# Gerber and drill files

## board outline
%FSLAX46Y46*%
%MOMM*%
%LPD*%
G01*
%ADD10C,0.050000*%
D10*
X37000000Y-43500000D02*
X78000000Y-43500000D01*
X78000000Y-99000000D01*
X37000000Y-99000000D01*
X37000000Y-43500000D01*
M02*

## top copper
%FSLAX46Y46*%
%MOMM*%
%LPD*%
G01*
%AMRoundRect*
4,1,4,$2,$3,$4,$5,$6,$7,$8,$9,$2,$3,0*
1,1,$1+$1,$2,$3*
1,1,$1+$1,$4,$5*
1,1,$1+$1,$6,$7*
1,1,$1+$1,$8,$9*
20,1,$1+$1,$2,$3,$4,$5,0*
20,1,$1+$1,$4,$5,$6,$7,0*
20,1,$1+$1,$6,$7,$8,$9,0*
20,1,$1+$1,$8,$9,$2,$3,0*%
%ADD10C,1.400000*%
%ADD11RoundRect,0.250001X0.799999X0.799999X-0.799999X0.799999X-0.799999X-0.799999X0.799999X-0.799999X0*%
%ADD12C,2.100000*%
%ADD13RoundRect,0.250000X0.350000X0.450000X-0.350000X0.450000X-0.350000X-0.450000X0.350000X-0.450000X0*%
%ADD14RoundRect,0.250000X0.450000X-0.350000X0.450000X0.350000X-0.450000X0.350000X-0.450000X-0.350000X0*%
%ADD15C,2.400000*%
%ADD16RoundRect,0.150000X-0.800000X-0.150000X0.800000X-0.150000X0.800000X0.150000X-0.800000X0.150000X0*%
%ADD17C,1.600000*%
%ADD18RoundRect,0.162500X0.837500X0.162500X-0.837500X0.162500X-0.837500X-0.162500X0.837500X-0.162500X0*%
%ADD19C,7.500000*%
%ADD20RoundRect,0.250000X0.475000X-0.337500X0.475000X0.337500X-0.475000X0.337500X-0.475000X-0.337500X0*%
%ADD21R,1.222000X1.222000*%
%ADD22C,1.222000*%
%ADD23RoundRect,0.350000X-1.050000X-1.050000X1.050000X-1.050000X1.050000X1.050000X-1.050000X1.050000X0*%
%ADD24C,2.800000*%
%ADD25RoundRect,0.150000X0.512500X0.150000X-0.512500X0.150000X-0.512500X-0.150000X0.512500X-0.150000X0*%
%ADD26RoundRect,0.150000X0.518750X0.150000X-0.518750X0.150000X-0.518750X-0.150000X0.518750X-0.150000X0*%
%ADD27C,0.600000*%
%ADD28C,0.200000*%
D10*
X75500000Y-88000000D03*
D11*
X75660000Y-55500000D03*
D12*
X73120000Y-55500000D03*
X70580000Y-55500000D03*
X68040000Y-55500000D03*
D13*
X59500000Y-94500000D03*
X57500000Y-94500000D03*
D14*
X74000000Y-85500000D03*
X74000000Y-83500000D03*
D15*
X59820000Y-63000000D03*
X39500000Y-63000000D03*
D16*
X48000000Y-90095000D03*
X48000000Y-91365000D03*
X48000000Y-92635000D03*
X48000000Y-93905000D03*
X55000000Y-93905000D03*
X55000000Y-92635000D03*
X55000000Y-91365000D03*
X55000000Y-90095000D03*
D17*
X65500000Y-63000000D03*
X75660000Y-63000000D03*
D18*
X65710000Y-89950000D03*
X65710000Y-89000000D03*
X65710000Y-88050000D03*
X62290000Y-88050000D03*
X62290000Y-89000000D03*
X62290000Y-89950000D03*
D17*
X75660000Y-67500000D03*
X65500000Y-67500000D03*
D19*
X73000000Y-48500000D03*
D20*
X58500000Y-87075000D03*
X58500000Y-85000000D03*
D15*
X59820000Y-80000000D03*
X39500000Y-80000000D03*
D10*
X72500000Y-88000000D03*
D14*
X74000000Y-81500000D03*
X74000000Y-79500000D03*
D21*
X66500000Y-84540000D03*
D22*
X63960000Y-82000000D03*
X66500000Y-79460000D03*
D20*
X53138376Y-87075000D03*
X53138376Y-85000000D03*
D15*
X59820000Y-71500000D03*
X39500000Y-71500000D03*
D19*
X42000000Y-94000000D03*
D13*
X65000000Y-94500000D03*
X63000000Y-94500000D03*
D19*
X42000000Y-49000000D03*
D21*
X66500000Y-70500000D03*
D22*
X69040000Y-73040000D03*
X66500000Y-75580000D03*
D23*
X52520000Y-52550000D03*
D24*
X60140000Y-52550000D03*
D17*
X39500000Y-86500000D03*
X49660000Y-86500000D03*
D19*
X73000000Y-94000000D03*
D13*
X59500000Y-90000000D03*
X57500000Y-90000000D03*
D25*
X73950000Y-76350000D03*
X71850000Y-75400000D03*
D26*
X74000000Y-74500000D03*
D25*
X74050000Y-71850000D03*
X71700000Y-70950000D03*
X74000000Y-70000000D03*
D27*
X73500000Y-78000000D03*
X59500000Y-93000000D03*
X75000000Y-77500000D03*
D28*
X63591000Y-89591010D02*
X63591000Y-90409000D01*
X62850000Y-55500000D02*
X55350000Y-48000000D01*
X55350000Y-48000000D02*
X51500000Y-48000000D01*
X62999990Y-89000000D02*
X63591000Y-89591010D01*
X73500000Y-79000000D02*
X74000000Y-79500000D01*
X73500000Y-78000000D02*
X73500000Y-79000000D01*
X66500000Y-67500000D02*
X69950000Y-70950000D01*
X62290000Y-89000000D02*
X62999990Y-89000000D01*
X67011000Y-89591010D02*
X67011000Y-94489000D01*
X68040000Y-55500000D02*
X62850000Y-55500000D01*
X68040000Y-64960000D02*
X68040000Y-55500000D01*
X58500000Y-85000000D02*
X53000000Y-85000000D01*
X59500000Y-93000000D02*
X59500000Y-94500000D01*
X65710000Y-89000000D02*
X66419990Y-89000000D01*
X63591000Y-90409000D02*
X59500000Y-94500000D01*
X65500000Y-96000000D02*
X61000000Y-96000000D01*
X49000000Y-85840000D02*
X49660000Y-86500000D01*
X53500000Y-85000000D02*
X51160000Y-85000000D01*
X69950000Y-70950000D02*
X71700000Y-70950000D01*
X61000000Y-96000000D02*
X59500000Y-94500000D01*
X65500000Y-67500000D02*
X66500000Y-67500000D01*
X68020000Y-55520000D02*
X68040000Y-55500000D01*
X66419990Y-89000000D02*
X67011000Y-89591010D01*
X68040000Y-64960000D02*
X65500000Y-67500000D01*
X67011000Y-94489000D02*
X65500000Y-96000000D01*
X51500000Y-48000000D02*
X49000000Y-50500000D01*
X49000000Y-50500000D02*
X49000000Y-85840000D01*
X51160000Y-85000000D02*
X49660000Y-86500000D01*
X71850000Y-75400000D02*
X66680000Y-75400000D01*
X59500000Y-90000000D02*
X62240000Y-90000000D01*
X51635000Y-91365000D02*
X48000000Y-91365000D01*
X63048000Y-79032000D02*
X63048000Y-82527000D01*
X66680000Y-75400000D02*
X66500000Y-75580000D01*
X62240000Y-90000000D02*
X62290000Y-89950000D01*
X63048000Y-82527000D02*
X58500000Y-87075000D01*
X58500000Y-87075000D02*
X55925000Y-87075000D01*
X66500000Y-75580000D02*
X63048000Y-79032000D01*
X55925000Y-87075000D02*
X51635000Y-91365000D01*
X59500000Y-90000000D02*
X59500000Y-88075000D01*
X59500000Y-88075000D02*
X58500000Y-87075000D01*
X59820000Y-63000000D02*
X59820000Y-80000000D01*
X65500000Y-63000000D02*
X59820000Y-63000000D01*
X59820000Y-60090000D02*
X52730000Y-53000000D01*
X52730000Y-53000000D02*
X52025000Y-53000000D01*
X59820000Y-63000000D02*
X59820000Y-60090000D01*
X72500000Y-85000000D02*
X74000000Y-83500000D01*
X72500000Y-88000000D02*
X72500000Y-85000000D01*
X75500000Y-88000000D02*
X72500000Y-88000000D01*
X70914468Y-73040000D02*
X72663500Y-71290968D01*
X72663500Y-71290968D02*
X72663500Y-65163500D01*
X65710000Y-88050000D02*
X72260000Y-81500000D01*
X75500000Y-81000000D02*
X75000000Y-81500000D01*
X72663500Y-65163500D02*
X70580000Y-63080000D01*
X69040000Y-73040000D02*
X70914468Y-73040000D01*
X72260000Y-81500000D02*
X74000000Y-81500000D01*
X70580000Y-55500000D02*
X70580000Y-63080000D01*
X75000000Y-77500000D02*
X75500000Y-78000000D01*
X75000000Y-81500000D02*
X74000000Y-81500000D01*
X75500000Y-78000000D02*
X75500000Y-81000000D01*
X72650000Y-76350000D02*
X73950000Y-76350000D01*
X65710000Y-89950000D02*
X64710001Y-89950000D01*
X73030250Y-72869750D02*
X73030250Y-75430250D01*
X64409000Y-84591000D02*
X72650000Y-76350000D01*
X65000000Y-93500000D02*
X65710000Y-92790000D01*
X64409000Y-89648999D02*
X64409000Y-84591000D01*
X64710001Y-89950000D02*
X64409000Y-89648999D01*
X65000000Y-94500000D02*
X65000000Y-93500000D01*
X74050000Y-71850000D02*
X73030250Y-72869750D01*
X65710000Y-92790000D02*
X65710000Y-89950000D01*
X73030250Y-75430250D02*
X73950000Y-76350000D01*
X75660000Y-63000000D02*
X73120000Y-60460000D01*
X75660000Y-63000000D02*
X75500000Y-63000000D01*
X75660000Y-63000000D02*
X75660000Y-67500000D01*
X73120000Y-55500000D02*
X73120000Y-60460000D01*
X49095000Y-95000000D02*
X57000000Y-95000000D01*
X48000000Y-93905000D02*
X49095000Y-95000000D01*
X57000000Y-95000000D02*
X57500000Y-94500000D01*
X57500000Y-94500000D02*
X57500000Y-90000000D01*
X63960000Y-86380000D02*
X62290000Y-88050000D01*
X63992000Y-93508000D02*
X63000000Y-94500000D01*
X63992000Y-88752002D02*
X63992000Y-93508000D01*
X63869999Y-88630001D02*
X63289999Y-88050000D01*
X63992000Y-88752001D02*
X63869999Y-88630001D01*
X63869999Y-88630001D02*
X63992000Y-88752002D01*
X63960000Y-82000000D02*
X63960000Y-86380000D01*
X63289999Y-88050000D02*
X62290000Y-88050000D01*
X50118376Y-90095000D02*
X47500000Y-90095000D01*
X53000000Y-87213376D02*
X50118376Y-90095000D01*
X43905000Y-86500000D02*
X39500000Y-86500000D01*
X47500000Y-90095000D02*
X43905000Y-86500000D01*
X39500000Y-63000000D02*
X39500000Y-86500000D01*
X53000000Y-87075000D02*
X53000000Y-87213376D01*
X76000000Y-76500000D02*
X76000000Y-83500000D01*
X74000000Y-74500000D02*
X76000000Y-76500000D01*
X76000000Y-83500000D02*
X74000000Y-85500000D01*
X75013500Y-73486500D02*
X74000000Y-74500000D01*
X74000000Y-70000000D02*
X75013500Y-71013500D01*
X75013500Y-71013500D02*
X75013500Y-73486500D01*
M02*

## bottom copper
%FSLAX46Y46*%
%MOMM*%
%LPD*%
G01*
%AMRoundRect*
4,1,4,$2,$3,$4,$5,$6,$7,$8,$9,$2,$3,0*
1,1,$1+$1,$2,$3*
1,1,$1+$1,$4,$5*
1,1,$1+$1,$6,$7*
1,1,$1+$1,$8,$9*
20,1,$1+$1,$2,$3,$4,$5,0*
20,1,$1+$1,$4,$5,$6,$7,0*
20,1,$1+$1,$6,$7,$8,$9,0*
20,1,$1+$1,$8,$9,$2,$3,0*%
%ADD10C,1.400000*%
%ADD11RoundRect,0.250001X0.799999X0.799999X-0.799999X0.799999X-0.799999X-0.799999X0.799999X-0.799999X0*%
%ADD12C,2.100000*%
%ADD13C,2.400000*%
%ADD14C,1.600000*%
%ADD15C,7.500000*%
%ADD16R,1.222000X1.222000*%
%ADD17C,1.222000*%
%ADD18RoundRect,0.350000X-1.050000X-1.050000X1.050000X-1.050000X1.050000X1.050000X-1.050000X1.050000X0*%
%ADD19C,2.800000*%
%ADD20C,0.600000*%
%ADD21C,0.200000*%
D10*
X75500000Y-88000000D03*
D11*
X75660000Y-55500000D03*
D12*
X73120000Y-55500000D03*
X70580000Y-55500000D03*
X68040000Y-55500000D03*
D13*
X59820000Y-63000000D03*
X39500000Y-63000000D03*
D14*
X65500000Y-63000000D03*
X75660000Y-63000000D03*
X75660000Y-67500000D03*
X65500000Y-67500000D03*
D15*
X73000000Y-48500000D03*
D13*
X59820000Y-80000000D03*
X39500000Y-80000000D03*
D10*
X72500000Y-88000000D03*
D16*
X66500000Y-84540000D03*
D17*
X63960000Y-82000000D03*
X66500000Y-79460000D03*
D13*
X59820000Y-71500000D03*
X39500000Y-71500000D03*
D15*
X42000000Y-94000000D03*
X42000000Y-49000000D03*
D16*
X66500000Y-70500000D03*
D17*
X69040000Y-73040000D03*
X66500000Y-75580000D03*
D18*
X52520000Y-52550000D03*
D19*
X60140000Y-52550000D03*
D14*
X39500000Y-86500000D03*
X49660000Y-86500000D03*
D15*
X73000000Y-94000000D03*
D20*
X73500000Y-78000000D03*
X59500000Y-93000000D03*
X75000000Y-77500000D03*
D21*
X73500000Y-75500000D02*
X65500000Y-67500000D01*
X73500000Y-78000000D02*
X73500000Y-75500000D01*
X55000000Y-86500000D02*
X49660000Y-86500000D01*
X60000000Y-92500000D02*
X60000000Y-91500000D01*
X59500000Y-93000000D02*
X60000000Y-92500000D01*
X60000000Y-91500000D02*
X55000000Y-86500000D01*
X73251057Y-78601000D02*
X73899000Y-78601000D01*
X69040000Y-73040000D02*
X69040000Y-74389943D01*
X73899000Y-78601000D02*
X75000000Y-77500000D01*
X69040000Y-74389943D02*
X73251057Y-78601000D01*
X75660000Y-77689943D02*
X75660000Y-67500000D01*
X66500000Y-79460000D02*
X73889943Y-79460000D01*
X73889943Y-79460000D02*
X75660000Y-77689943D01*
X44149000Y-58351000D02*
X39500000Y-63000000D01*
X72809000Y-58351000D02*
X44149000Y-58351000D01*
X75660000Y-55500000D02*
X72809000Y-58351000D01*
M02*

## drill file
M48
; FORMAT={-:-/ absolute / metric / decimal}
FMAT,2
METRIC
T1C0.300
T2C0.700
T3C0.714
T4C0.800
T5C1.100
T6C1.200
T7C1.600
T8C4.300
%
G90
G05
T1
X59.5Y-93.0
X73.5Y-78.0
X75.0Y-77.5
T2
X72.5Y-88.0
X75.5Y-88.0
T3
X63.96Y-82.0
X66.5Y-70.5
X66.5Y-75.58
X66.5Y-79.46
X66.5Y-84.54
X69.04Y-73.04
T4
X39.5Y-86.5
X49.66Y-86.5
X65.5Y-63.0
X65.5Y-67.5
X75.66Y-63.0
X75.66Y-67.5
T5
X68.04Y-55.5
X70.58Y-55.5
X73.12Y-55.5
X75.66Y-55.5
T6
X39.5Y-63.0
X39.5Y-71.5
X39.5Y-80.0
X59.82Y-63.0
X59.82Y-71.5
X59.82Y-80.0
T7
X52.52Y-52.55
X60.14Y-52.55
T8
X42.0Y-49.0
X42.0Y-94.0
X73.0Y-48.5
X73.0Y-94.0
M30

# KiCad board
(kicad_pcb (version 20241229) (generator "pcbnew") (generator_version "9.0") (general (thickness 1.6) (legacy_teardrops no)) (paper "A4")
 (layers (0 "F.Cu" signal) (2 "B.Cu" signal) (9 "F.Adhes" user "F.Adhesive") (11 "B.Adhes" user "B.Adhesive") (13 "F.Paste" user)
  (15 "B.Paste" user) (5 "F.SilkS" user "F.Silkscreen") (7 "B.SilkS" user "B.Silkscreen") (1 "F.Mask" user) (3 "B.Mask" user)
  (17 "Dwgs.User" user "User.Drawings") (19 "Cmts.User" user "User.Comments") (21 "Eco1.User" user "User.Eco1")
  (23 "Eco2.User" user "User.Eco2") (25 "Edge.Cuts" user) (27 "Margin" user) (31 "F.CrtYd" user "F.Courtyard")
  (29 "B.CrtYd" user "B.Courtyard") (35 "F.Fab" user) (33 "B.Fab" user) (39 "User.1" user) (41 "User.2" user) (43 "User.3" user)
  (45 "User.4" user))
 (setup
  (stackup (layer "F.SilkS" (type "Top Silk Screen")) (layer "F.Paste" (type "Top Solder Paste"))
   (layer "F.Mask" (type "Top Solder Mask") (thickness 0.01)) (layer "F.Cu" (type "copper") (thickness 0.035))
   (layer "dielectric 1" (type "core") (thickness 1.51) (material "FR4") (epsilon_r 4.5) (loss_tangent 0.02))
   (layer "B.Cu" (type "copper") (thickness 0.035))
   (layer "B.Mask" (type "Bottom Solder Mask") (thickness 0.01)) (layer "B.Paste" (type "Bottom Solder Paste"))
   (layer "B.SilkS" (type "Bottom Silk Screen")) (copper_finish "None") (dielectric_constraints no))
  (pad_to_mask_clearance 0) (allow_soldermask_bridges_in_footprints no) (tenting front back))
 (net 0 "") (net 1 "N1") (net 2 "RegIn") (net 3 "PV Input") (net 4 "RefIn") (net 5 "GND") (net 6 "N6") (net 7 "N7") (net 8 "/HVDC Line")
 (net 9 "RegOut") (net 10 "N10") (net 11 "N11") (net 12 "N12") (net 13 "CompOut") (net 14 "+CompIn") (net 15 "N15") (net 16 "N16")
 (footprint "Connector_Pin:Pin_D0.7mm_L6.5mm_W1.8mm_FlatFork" (layer "F.Cu") (at 75.5 88)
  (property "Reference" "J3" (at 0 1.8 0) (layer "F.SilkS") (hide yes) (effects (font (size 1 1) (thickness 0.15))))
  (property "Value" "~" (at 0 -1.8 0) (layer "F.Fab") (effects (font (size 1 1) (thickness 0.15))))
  (pad "1" thru_hole circle (at 0 0) (size 1.4 1.4) (drill 0.7) (layers "*.Cu" "*.Mask") (remove_unused_layers no) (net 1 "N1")))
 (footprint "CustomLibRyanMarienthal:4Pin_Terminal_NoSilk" (layer "F.Cu") (at 71.85 55.54 180)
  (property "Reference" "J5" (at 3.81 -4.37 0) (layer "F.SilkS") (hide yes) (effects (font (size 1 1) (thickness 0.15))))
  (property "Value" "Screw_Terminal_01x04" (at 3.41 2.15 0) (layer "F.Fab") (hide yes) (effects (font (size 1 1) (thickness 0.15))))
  (pad "1" thru_hole roundrect (at -3.81 0.04 180) (size 2.1 2.1) (drill 1.1) (layers "*.Cu" "*.Mask") (remove_unused_layers no)
   (roundrect_rratio 0.119048) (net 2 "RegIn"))
  (pad "2" thru_hole circle (at -1.27 0.04 180) (size 2.1 2.1) (drill 1.1) (layers "*.Cu" "*.Mask") (remove_unused_layers no)
   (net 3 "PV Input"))
  (pad "3" thru_hole circle (at 1.27 0.04 180) (size 2.1 2.1) (drill 1.1) (layers "*.Cu" "*.Mask") (remove_unused_layers no) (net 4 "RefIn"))
  (pad "4" thru_hole circle (at 3.81 0.04 180) (size 2.1 2.1) (drill 1.1) (layers "*.Cu" "*.Mask") (remove_unused_layers no) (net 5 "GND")))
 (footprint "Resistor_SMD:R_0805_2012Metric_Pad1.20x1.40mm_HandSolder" (layer "F.Cu") (at 58.5 94.5 180)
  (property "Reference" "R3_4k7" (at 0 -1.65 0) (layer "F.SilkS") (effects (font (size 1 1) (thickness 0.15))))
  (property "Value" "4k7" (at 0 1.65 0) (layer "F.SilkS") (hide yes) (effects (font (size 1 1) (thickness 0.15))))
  (pad "1" smd roundrect (at -1 0 180) (size 1.2 1.4) (layers "F.Cu" "F.Mask" "F.Paste") (roundrect_rratio 0.208333) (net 5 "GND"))
  (pad "2" smd roundrect (at 1 0 180) (size 1.2 1.4) (layers "F.Cu" "F.Mask" "F.Paste") (roundrect_rratio 0.208333) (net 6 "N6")))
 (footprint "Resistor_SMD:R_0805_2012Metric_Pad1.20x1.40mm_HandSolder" (layer "F.Cu") (at 74 84.5 90)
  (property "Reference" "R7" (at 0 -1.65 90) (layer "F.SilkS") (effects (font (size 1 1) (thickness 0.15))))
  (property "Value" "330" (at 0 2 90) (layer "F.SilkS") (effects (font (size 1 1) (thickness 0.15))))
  (pad "1" smd roundrect (at -1 0 90) (size 1.2 1.4) (layers "F.Cu" "F.Mask" "F.Paste") (roundrect_rratio 0.208333) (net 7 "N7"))
  (pad "2" smd roundrect (at 1 0 90) (size 1.2 1.4) (layers "F.Cu" "F.Mask" "F.Paste") (roundrect_rratio 0.208333) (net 1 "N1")))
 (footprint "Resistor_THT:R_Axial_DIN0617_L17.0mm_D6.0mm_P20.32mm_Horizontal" (layer "F.Cu") (at 59.82 63 180)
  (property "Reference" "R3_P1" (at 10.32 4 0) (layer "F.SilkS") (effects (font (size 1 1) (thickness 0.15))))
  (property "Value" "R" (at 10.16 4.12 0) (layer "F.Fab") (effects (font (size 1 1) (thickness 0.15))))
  (pad "1" thru_hole circle (at 0 0 180) (size 2.4 2.4) (drill 1.2) (layers "*.Cu" "*.Mask") (remove_unused_layers no) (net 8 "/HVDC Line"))
  (pad "2" thru_hole circle (at 20.32 0 180) (size 2.4 2.4) (drill 1.2) (layers "*.Cu" "*.Mask") (remove_unused_layers no) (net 2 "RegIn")))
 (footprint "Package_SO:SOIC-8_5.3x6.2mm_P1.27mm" (layer "F.Cu") (at 51.5 92)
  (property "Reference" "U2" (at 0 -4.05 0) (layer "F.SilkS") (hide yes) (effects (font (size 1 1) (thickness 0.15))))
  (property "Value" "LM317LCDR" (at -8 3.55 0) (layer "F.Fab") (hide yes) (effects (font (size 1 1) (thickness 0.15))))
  (pad "1" smd roundrect (at -3.5 -1.905) (size 1.9 0.6) (layers "F.Cu" "F.Mask" "F.Paste") (roundrect_rratio 0.25) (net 2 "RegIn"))
  (pad "2" smd roundrect (at -3.5 -0.635) (size 1.9 0.6) (layers "F.Cu" "F.Mask" "F.Paste") (roundrect_rratio 0.25) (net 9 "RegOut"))
  (pad "3" smd roundrect (at -3.5 0.635) (size 1.9 0.6) (layers "F.Cu" "F.Mask" "F.Paste") (roundrect_rratio 0.25) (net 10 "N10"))
  (pad "4" smd roundrect (at -3.5 1.905) (size 1.9 0.6) (layers "F.Cu" "F.Mask" "F.Paste") (roundrect_rratio 0.25) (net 6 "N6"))
  (pad "5" smd roundrect (at 3.5 1.905) (size 1.9 0.6) (layers "F.Cu" "F.Mask" "F.Paste") (roundrect_rratio 0.25))
  (pad "6" smd roundrect (at 3.5 0.635) (size 1.9 0.6) (layers "F.Cu" "F.Mask" "F.Paste") (roundrect_rratio 0.25) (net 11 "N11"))
  (pad "7" smd roundrect (at 3.5 -0.635) (size 1.9 0.6) (layers "F.Cu" "F.Mask" "F.Paste") (roundrect_rratio 0.25) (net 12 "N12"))
  (pad "8" smd roundrect (at 3.5 -1.905) (size 1.9 0.6) (layers "F.Cu" "F.Mask" "F.Paste") (roundrect_rratio 0.25)))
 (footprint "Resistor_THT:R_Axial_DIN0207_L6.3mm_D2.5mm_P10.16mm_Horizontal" (layer "F.Cu") (at 65.5 63)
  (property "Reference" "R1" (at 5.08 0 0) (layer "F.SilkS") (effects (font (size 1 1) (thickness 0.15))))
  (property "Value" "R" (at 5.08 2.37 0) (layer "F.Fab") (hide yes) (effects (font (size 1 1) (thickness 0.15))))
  (pad "1" thru_hole circle (at 0 0) (size 1.6 1.6) (drill 0.8) (layers "*.Cu" "*.Mask") (remove_unused_layers no) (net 8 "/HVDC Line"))
  (pad "2" thru_hole circle (at 10.16 0) (size 1.6 1.6) (drill 0.8) (layers "*.Cu" "*.Mask") (remove_unused_layers no) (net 3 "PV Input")))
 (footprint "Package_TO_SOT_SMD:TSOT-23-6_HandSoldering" (layer "F.Cu") (at 64 89 180)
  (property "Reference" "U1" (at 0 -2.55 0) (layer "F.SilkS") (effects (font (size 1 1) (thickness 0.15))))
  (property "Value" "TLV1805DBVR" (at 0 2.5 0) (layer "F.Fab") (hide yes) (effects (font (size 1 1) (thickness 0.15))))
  (pad "1" smd roundrect (at -1.71 -0.95 180) (size 2 0.65) (layers "F.Cu" "F.Mask" "F.Paste") (roundrect_rratio 0.25) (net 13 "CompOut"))
  (pad "2" smd roundrect (at -1.71 0 180) (size 2 0.65) (layers "F.Cu" "F.Mask" "F.Paste") (roundrect_rratio 0.25) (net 5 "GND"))
  (pad "3" smd roundrect (at -1.71 0.95 180) (size 2 0.65) (layers "F.Cu" "F.Mask" "F.Paste") (roundrect_rratio 0.25) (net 4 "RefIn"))
  (pad "4" smd roundrect (at 1.71 0.95 180) (size 2 0.65) (layers "F.Cu" "F.Mask" "F.Paste") (roundrect_rratio 0.25) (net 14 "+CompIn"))
  (pad "5" smd roundrect (at 1.71 0 180) (size 2 0.65) (layers "F.Cu" "F.Mask" "F.Paste") (roundrect_rratio 0.25) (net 5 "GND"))
  (pad "6" smd roundrect (at 1.71 -0.95 180) (size 2 0.65) (layers "F.Cu" "F.Mask" "F.Paste") (roundrect_rratio 0.25) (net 9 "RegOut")))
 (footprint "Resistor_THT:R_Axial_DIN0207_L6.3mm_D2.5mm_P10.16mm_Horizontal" (layer "F.Cu") (at 75.66 67.5 180)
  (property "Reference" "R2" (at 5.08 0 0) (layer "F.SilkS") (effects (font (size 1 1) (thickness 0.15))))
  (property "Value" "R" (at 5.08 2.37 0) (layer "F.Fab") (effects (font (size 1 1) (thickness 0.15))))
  (pad "1" thru_hole circle (at 0 0 180) (size 1.6 1.6) (drill 0.8) (layers "*.Cu" "*.Mask") (remove_unused_layers no) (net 3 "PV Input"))
  (pad "2" thru_hole circle (at 10.16 0 180) (size 1.6 1.6) (drill 0.8) (layers "*.Cu" "*.Mask") (remove_unused_layers no) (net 5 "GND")))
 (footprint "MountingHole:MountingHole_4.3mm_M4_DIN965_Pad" (layer "F.Cu") (at 73 48.5)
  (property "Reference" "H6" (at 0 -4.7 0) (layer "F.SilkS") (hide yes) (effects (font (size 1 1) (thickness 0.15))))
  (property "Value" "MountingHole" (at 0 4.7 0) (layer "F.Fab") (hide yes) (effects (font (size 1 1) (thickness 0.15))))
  (pad "1" thru_hole circle (at 0 0) (size 7.5 7.5) (drill 4.3) (layers "*.Cu" "*.Mask") (remove_unused_layers no) (zone_connect 2)))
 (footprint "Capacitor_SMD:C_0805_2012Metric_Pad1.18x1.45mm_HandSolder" (layer "F.Cu") (at 58.5 86.0375 90)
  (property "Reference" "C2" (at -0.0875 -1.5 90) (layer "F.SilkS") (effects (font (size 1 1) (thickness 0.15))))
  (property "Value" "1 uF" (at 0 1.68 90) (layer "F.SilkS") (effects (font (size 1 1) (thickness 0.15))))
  (pad "1" smd roundrect (at -1.0375 0 90) (size 1.175 1.45) (layers "F.Cu" "F.Mask" "F.Paste") (roundrect_rratio 0.212766) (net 9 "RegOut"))
  (pad "2" smd roundrect (at 1.0375 0 90) (size 1.175 1.45) (layers "F.Cu" "F.Mask" "F.Paste") (roundrect_rratio 0.212766) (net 5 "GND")))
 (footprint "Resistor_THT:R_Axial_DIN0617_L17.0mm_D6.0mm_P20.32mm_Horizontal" (layer "F.Cu") (at 59.82 80 180)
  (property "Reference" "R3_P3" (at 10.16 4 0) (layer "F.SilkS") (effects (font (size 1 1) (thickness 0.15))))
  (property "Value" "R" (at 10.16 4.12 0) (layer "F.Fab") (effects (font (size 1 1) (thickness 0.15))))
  (pad "1" thru_hole circle (at 0 0 180) (size 2.4 2.4) (drill 1.2) (layers "*.Cu" "*.Mask") (remove_unused_layers no) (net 8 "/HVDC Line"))
  (pad "2" thru_hole circle (at 20.32 0 180) (size 2.4 2.4) (drill 1.2) (layers "*.Cu" "*.Mask") (remove_unused_layers no) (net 2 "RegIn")))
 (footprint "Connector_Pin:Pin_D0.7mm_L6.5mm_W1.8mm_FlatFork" (layer "F.Cu") (at 72.5 88)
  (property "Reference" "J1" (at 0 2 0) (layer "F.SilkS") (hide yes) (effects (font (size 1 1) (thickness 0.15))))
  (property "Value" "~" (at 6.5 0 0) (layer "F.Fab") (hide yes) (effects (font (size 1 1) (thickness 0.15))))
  (pad "1" thru_hole circle (at 0 0) (size 1.4 1.4) (drill 0.7) (layers "*.Cu" "*.Mask") (remove_unused_layers no) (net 1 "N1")))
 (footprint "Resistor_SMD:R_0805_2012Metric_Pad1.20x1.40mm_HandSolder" (layer "F.Cu") (at 74 80.5 90)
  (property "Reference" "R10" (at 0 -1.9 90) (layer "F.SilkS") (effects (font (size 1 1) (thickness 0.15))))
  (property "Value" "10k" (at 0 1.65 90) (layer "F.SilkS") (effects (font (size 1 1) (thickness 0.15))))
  (pad "1" smd roundrect (at -1 0 90) (size 1.2 1.4) (layers "F.Cu" "F.Mask" "F.Paste") (roundrect_rratio 0.208333) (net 4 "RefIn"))
  (pad "2" smd roundrect (at 1 0 90) (size 1.2 1.4) (layers "F.Cu" "F.Mask" "F.Paste") (roundrect_rratio 0.208333) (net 5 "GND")))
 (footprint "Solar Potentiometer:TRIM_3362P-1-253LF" (layer "F.Cu") (at 66.5 82 90)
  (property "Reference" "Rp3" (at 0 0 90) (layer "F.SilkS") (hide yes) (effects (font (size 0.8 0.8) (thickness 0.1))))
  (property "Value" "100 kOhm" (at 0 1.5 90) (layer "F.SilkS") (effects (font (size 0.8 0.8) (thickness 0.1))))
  (pad "1" thru_hole rect (at -2.54 0 90) (size 1.222 1.222) (drill 0.714) (layers "*.Cu" "*.Mask") (remove_unused_layers no) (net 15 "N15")
   (solder_mask_margin 0.102))
  (pad "2" thru_hole circle (at 0 -2.54 90) (size 1.222 1.222) (drill 0.714) (layers "*.Cu" "*.Mask") (remove_unused_layers no)
   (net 14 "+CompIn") (solder_mask_margin 0.102))
  (pad "3" thru_hole circle (at 2.54 0 90) (size 1.222 1.222) (drill 0.714) (layers "*.Cu" "*.Mask") (remove_unused_layers no)
   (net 3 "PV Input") (solder_mask_margin 0.102)))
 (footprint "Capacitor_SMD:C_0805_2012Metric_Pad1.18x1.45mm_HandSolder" (layer "F.Cu") (at 53.138376 86.0375 90)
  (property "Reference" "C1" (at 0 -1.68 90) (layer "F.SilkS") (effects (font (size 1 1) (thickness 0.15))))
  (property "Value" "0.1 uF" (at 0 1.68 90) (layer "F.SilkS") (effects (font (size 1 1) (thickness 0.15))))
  (pad "1" smd roundrect (at -1.0375 0 90) (size 1.175 1.45) (layers "F.Cu" "F.Mask" "F.Paste") (roundrect_rratio 0.212766) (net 2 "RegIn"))
  (pad "2" smd roundrect (at 1.0375 0 90) (size 1.175 1.45) (layers "F.Cu" "F.Mask" "F.Paste") (roundrect_rratio 0.212766) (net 5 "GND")))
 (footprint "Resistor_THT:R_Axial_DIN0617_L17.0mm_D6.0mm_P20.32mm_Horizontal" (layer "F.Cu") (at 59.82 71.5 180)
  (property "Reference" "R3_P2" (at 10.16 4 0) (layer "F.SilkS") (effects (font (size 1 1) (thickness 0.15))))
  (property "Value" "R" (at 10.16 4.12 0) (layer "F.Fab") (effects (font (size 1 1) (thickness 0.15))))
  (pad "1" thru_hole circle (at 0 0 180) (size 2.4 2.4) (drill 1.2) (layers "*.Cu" "*.Mask") (remove_unused_layers no) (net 8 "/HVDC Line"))
  (pad "2" thru_hole circle (at 20.32 0 180) (size 2.4 2.4) (drill 1.2) (layers "*.Cu" "*.Mask") (remove_unused_layers no) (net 2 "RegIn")))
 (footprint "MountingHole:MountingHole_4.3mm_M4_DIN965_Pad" (layer "F.Cu") (at 42 94)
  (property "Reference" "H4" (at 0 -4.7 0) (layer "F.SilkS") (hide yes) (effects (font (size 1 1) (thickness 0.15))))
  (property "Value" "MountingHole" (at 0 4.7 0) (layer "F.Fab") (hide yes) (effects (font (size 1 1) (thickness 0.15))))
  (pad "1" thru_hole circle (at 0 0) (size 7.5 7.5) (drill 4.3) (layers "*.Cu" "*.Mask") (remove_unused_layers no) (zone_connect 2)))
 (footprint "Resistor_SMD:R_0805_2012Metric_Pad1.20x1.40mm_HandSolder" (layer "F.Cu") (at 64 94.5 180)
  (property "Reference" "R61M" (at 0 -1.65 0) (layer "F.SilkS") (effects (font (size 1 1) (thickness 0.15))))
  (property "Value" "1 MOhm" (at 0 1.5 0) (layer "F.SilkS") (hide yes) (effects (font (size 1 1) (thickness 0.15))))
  (pad "1" smd roundrect (at -1 0 180) (size 1.2 1.4) (layers "F.Cu" "F.Mask" "F.Paste") (roundrect_rratio 0.208333) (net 13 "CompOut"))
  (pad "2" smd roundrect (at 1 0 180) (size 1.2 1.4) (layers "F.Cu" "F.Mask" "F.Paste") (roundrect_rratio 0.208333) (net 14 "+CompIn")))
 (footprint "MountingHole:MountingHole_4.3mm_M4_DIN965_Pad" (layer "F.Cu") (at 42 49)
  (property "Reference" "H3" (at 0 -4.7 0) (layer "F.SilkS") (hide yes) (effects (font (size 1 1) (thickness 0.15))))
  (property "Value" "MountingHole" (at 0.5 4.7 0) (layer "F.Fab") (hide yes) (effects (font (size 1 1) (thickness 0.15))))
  (pad "1" thru_hole circle (at 0 0) (size 7.5 7.5) (drill 4.3) (layers "*.Cu" "*.Mask") (remove_unused_layers no) (zone_connect 2)))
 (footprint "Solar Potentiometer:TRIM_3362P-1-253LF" (layer "F.Cu") (at 66.5 73.04 -90)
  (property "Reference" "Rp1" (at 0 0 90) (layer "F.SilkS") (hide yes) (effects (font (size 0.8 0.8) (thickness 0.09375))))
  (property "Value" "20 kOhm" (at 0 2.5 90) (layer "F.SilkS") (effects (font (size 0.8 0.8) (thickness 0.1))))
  (pad "1" thru_hole rect (at -2.54 0 270) (size 1.222 1.222) (drill 0.714) (layers "*.Cu" "*.Mask") (remove_unused_layers no)
   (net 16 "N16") (solder_mask_margin 0.102))
  (pad "2" thru_hole circle (at 0 -2.54 270) (size 1.222 1.222) (drill 0.714) (layers "*.Cu" "*.Mask") (remove_unused_layers no)
   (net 4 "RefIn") (solder_mask_margin 0.102))
  (pad "3" thru_hole circle (at 2.54 0 270) (size 1.222 1.222) (drill 0.714) (layers "*.Cu" "*.Mask") (remove_unused_layers no)
   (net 9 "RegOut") (solder_mask_margin 0.102)))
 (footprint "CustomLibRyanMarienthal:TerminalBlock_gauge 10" (layer "F.Cu") (at 56.5 51)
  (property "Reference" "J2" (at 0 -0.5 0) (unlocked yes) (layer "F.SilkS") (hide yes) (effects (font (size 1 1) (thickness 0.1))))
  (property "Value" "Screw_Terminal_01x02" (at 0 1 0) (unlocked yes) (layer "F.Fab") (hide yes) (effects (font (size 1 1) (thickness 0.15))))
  (pad "1" thru_hole roundrect (at -3.98 1.55) (size 2.8 2.8) (drill 1.6) (layers "*.Cu" "*.Mask") (remove_unused_layers no)
   (roundrect_rratio 0.125) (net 8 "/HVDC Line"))
  (pad "2" thru_hole circle (at 3.64 1.55) (size 2.8 2.8) (drill 1.6) (layers "*.Cu" "*.Mask") (remove_unused_layers no) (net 5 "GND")))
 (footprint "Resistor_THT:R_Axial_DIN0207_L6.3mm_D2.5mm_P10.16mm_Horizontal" (layer "F.Cu") (at 39.5 86.5)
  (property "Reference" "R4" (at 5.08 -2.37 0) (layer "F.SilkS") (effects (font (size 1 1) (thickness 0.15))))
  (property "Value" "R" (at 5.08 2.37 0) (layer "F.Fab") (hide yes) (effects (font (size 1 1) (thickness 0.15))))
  (pad "1" thru_hole circle (at 0 0) (size 1.6 1.6) (drill 0.8) (layers "*.Cu" "*.Mask") (remove_unused_layers no) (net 2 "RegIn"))
  (pad "2" thru_hole circle (at 10.16 0) (size 1.6 1.6) (drill 0.8) (layers "*.Cu" "*.Mask") (remove_unused_layers no) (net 5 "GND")))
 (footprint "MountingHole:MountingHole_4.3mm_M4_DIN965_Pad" (layer "F.Cu") (at 73 94)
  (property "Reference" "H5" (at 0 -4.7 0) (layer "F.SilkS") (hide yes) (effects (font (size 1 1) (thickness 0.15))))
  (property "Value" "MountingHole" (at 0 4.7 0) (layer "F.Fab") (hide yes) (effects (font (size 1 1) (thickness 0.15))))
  (pad "1" thru_hole circle (at 0 0) (size 7.5 7.5) (drill 4.3) (layers "*.Cu" "*.Mask") (remove_unused_layers no) (zone_connect 2)))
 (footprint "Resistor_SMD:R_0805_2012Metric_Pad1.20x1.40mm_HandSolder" (layer "F.Cu") (at 58.5 90 180)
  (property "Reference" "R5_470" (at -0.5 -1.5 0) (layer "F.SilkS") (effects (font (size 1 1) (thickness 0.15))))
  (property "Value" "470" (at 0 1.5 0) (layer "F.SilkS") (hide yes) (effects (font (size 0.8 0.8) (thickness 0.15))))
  (pad "1" smd roundrect (at -1 0 180) (size 1.2 1.4) (layers "F.Cu" "F.Mask" "F.Paste") (roundrect_rratio 0.208333) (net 9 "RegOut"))
  (pad "2" smd roundrect (at 1 0 180) (size 1.2 1.4) (layers "F.Cu" "F.Mask" "F.Paste") (roundrect_rratio 0.208333) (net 6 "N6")))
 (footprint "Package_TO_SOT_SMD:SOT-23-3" (layer "F.Cu") (at 72.8 75.4 180)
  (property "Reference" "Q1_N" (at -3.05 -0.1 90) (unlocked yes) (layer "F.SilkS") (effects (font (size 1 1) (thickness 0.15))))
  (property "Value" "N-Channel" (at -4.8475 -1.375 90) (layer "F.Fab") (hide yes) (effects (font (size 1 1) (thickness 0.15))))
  (pad "1" smd roundrect (at -1.15 -0.95 180) (size 1.325 0.6) (layers "F.Cu" "F.Mask" "F.Paste") (roundrect_rratio 0.25) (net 13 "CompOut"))
  (pad "2" smd roundrect (at 0.95 0 180) (size 1.325 0.6) (layers "F.Cu" "F.Mask" "F.Paste") (roundrect_rratio 0.25) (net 9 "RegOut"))
  (pad "3" smd roundrect (at -1.2 0.9 180) (size 1.3375 0.6) (layers "F.Cu" "F.Mask" "F.Paste") (roundrect_rratio 0.25) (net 7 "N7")))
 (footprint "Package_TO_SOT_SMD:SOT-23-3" (layer "F.Cu") (at 72.85 70.95 180)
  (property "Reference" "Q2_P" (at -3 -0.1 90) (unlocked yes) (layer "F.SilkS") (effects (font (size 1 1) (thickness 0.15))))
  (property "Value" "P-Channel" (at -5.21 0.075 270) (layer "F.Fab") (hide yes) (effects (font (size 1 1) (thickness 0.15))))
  (pad "1" smd roundrect (at -1.2 -0.9 180) (size 1.325 0.6) (layers "F.Cu" "F.Mask" "F.Paste") (roundrect_rratio 0.25) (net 13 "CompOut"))
  (pad "2" smd roundrect (at 1.15 0 180) (size 1.325 0.6) (layers "F.Cu" "F.Mask" "F.Paste") (roundrect_rratio 0.25) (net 5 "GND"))
  (pad "3" smd roundrect (at -1.15 0.95 180) (size 1.325 0.6) (layers "F.Cu" "F.Mask" "F.Paste") (roundrect_rratio 0.25) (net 7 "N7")))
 (gr_rect (start 37 43.5) (end 78 99) (stroke (width 0.05) (type default)) (fill no) (layer "Edge.Cuts"))
 (segment (start 63.591 89.59101) (end 63.591 90.409) (width 0.2) (layer "F.Cu") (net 5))
 (segment (start 62.85 55.5) (end 55.35 48) (width 0.2) (layer "F.Cu") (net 5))
 (segment (start 55.35 48) (end 51.5 48) (width 0.2) (layer "F.Cu") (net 5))
 (segment (start 62.99999 89) (end 63.591 89.59101) (width 0.2) (layer "F.Cu") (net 5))
 (segment (start 73.5 79) (end 74 79.5) (width 0.2) (layer "F.Cu") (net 5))
 (segment (start 73.5 78) (end 73.5 79) (width 0.2) (layer "F.Cu") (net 5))
 (segment (start 66.5 67.5) (end 69.95 70.95) (width 0.2) (layer "F.Cu") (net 5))
 (segment (start 62.29 89) (end 62.99999 89) (width 0.2) (layer "F.Cu") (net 5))
 (segment (start 67.011 89.59101) (end 67.011 94.489) (width 0.2) (layer "F.Cu") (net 5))
 (segment (start 68.04 55.5) (end 62.85 55.5) (width 0.2) (layer "F.Cu") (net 5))
 (segment (start 68.04 64.96) (end 68.04 55.5) (width 0.2) (layer "F.Cu") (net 5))
 (segment (start 58.5 85) (end 53 85) (width 0.2) (layer "F.Cu") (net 5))
 (segment (start 59.5 93) (end 59.5 94.5) (width 0.2) (layer "F.Cu") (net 5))
 (segment (start 65.71 89) (end 66.41999 89) (width 0.2) (layer "F.Cu") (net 5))
 (segment (start 63.591 90.409) (end 59.5 94.5) (width 0.2) (layer "F.Cu") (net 5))
 (segment (start 65.5 96) (end 61 96) (width 0.2) (layer "F.Cu") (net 5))
 (segment (start 49 85.84) (end 49.66 86.5) (width 0.2) (layer "F.Cu") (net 5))
 (segment (start 53.5 85) (end 51.16 85) (width 0.2) (layer "F.Cu") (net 5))
 (segment (start 69.95 70.95) (end 71.7 70.95) (width 0.2) (layer "F.Cu") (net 5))
 (segment (start 61 96) (end 59.5 94.5) (width 0.2) (layer "F.Cu") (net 5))
 (segment (start 65.5 67.5) (end 66.5 67.5) (width 0.2) (layer "F.Cu") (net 5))
 (segment (start 68.02 55.52) (end 68.04 55.5) (width 0.2) (layer "F.Cu") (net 5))
 (segment (start 66.41999 89) (end 67.011 89.59101) (width 0.2) (layer "F.Cu") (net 5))
 (segment (start 68.04 64.96) (end 65.5 67.5) (width 0.2) (layer "F.Cu") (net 5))
 (segment (start 67.011 94.489) (end 65.5 96) (width 0.2) (layer "F.Cu") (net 5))
 (segment (start 51.5 48) (end 49 50.5) (width 0.2) (layer "F.Cu") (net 5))
 (segment (start 49 50.5) (end 49 85.84) (width 0.2) (layer "F.Cu") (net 5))
 (segment (start 51.16 85) (end 49.66 86.5) (width 0.2) (layer "F.Cu") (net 5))
 (via (at 73.5 78) (size 0.6) (drill 0.3) (layers "F.Cu" "B.Cu") (free yes) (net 5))
 (via (at 59.5 93) (size 0.6) (drill 0.3) (layers "F.Cu" "B.Cu") (free yes) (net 5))
 (segment (start 73.5 75.5) (end 65.5 67.5) (width 0.2) (layer "B.Cu") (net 5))
 (segment (start 73.5 78) (end 73.5 75.5) (width 0.2) (layer "B.Cu") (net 5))
 (segment (start 55 86.5) (end 49.66 86.5) (width 0.2) (layer "B.Cu") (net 5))
 (segment (start 60 92.5) (end 60 91.5) (width 0.2) (layer "B.Cu") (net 5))
 (segment (start 59.5 93) (end 60 92.5) (width 0.2) (layer "B.Cu") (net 5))
 (segment (start 60 91.5) (end 55 86.5) (width 0.2) (layer "B.Cu") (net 5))
 (segment (start 71.85 75.4) (end 66.68 75.4) (width 0.2) (layer "F.Cu") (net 9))
 (segment (start 59.5 90) (end 62.24 90) (width 0.2) (layer "F.Cu") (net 9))
 (segment (start 51.635 91.365) (end 48 91.365) (width 0.2) (layer "F.Cu") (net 9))
 (segment (start 63.048 79.032) (end 63.048 82.527) (width 0.2) (layer "F.Cu") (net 9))
 (segment (start 66.68 75.4) (end 66.5 75.58) (width 0.2) (layer "F.Cu") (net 9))
 (segment (start 62.24 90) (end 62.29 89.95) (width 0.2) (layer "F.Cu") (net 9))
 (segment (start 63.048 82.527) (end 58.5 87.075) (width 0.2) (layer "F.Cu") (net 9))
 (segment (start 58.5 87.075) (end 55.925 87.075) (width 0.2) (layer "F.Cu") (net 9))
 (segment (start 66.5 75.58) (end 63.048 79.032) (width 0.2) (layer "F.Cu") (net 9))
 (segment (start 55.925 87.075) (end 51.635 91.365) (width 0.2) (layer "F.Cu") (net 9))
 (segment (start 59.5 90) (end 59.5 88.075) (width 0.2) (layer "F.Cu") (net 9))
 (segment (start 59.5 88.075) (end 58.5 87.075) (width 0.2) (layer "F.Cu") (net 9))
 (segment (start 59.82 63) (end 59.82 80) (width 0.2) (layer "F.Cu") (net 8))
 (segment (start 65.5 63) (end 59.82 63) (width 0.2) (layer "F.Cu") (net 8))
 (segment (start 59.82 60.09) (end 52.73 53) (width 0.2) (layer "F.Cu") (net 8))
 (segment (start 52.73 53) (end 52.025 53) (width 0.2) (layer "F.Cu") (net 8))
 (segment (start 59.82 63) (end 59.82 60.09) (width 0.2) (layer "F.Cu") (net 8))
 (segment (start 72.5 85) (end 74 83.5) (width 0.2) (layer "F.Cu") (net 1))
 (segment (start 72.5 88) (end 72.5 85) (width 0.2) (layer "F.Cu") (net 1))
 (segment (start 75.5 88) (end 72.5 88) (width 0.2) (layer "F.Cu") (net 1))
 (segment (start 70.914468 73.04) (end 72.6635 71.290968) (width 0.2) (layer "F.Cu") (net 4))
 (segment (start 72.6635 71.290968) (end 72.6635 65.1635) (width 0.2) (layer "F.Cu") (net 4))
 (segment (start 65.71 88.05) (end 72.26 81.5) (width 0.2) (layer "F.Cu") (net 4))
 (segment (start 75.5 81) (end 75 81.5) (width 0.2) (layer "F.Cu") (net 4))
 (segment (start 72.6635 65.1635) (end 70.58 63.08) (width 0.2) (layer "F.Cu") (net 4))
 (segment (start 69.04 73.04) (end 70.914468 73.04) (width 0.2) (layer "F.Cu") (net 4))
 (segment (start 72.26 81.5) (end 74 81.5) (width 0.2) (layer "F.Cu") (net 4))
 (segment (start 70.58 55.5) (end 70.58 63.08) (width 0.2) (layer "F.Cu") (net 4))
 (segment (start 75 77.5) (end 75.5 78) (width 0.2) (layer "F.Cu") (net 4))
 (segment (start 75 81.5) (end 74 81.5) (width 0.2) (layer "F.Cu") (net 4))
 (segment (start 75.5 78) (end 75.5 81) (width 0.2) (layer "F.Cu") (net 4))
 (via (at 75 77.5) (size 0.6) (drill 0.3) (layers "F.Cu" "B.Cu") (free yes) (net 4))
 (segment (start 73.251057 78.601) (end 73.899 78.601) (width 0.2) (layer "B.Cu") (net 4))
 (segment (start 69.04 73.04) (end 69.04 74.389943) (width 0.2) (layer "B.Cu") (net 4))
 (segment (start 73.899 78.601) (end 75 77.5) (width 0.2) (layer "B.Cu") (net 4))
 (segment (start 69.04 74.389943) (end 73.251057 78.601) (width 0.2) (layer "B.Cu") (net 4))
 (segment (start 72.65 76.35) (end 73.95 76.35) (width 0.2) (layer "F.Cu") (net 13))
 (segment (start 65.71 89.95) (end 64.710001 89.95) (width 0.2) (layer "F.Cu") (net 13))
 (segment (start 73.03025 72.86975) (end 73.03025 75.43025) (width 0.2) (layer "F.Cu") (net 13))
 (segment (start 64.409 84.591) (end 72.65 76.35) (width 0.2) (layer "F.Cu") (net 13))
 (segment (start 65 93.5) (end 65.71 92.79) (width 0.2) (layer "F.Cu") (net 13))
 (segment (start 64.409 89.648999) (end 64.409 84.591) (width 0.2) (layer "F.Cu") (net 13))
 (segment (start 64.710001 89.95) (end 64.409 89.648999) (width 0.2) (layer "F.Cu") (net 13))
 (segment (start 65 94.5) (end 65 93.5) (width 0.2) (layer "F.Cu") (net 13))
 (segment (start 74.05 71.85) (end 73.03025 72.86975) (width 0.2) (layer "F.Cu") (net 13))
 (segment (start 65.71 92.79) (end 65.71 89.95) (width 0.2) (layer "F.Cu") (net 13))
 (segment (start 73.03025 75.43025) (end 73.95 76.35) (width 0.2) (layer "F.Cu") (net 13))
 (segment (start 75.66 63) (end 73.12 60.46) (width 0.2) (layer "F.Cu") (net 3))
 (segment (start 75.66 63) (end 75.5 63) (width 0.2) (layer "F.Cu") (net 3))
 (segment (start 75.66 63) (end 75.66 67.5) (width 0.2) (layer "F.Cu") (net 3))
 (segment (start 73.12 55.5) (end 73.12 60.46) (width 0.2) (layer "F.Cu") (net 3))
 (segment (start 75.66 77.689943) (end 75.66 67.5) (width 0.2) (layer "B.Cu") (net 3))
 (segment (start 66.5 79.46) (end 73.889943 79.46) (width 0.2) (layer "B.Cu") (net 3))
 (segment (start 73.889943 79.46) (end 75.66 77.689943) (width 0.2) (layer "B.Cu") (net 3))
 (segment (start 49.095 95) (end 57 95) (width 0.2) (layer "F.Cu") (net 6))
 (segment (start 48 93.905) (end 49.095 95) (width 0.2) (layer "F.Cu") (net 6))
 (segment (start 57 95) (end 57.5 94.5) (width 0.2) (layer "F.Cu") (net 6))
 (segment (start 57.5 94.5) (end 57.5 90) (width 0.2) (layer "F.Cu") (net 6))
 (segment (start 63.96 86.38) (end 62.29 88.05) (width 0.2) (layer "F.Cu") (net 14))
 (segment (start 63.992 93.508) (end 63 94.5) (width 0.2) (layer "F.Cu") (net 14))
 (segment (start 63.992 88.752002) (end 63.992 93.508) (width 0.2) (layer "F.Cu") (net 14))
 (segment (start 63.869999 88.630001) (end 63.289999 88.05) (width 0.2) (layer "F.Cu") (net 14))
 (segment (start 63.992 88.752001) (end 63.869999 88.630001) (width 0.2) (layer "F.Cu") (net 14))
 (segment (start 63.869999 88.630001) (end 63.992 88.752002) (width 0.2) (layer "F.Cu") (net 14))
 (segment (start 63.96 82) (end 63.96 86.38) (width 0.2) (layer "F.Cu") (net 14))
 (segment (start 63.289999 88.05) (end 62.29 88.05) (width 0.2) (layer "F.Cu") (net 14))
 (segment (start 50.118376 90.095) (end 47.5 90.095) (width 0.2) (layer "F.Cu") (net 2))
 (segment (start 53 87.213376) (end 50.118376 90.095) (width 0.2) (layer "F.Cu") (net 2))
 (segment (start 43.905 86.5) (end 39.5 86.5) (width 0.2) (layer "F.Cu") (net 2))
 (segment (start 47.5 90.095) (end 43.905 86.5) (width 0.2) (layer "F.Cu") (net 2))
 (segment (start 39.5 63) (end 39.5 86.5) (width 0.2) (layer "F.Cu") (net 2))
 (segment (start 53 87.075) (end 53 87.213376) (width 0.2) (layer "F.Cu") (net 2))
 (segment (start 44.149 58.351) (end 39.5 63) (width 0.2) (layer "B.Cu") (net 2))
 (segment (start 72.809 58.351) (end 44.149 58.351) (width 0.2) (layer "B.Cu") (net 2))
 (segment (start 75.66 55.5) (end 72.809 58.351) (width 0.2) (layer "B.Cu") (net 2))
 (segment (start 76 76.5) (end 76 83.5) (width 0.2) (layer "F.Cu") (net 7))
 (segment (start 74 74.5) (end 76 76.5) (width 0.2) (layer "F.Cu") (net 7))
 (segment (start 76 83.5) (end 74 85.5) (width 0.2) (layer "F.Cu") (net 7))
 (segment (start 75.0135 73.4865) (end 74 74.5) (width 0.2) (layer "F.Cu") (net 7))
 (segment (start 74 70) (end 75.0135 71.0135) (width 0.2) (layer "F.Cu") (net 7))
 (segment (start 75.0135 71.0135) (end 75.0135 73.4865) (width 0.2) (layer "F.Cu") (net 7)))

